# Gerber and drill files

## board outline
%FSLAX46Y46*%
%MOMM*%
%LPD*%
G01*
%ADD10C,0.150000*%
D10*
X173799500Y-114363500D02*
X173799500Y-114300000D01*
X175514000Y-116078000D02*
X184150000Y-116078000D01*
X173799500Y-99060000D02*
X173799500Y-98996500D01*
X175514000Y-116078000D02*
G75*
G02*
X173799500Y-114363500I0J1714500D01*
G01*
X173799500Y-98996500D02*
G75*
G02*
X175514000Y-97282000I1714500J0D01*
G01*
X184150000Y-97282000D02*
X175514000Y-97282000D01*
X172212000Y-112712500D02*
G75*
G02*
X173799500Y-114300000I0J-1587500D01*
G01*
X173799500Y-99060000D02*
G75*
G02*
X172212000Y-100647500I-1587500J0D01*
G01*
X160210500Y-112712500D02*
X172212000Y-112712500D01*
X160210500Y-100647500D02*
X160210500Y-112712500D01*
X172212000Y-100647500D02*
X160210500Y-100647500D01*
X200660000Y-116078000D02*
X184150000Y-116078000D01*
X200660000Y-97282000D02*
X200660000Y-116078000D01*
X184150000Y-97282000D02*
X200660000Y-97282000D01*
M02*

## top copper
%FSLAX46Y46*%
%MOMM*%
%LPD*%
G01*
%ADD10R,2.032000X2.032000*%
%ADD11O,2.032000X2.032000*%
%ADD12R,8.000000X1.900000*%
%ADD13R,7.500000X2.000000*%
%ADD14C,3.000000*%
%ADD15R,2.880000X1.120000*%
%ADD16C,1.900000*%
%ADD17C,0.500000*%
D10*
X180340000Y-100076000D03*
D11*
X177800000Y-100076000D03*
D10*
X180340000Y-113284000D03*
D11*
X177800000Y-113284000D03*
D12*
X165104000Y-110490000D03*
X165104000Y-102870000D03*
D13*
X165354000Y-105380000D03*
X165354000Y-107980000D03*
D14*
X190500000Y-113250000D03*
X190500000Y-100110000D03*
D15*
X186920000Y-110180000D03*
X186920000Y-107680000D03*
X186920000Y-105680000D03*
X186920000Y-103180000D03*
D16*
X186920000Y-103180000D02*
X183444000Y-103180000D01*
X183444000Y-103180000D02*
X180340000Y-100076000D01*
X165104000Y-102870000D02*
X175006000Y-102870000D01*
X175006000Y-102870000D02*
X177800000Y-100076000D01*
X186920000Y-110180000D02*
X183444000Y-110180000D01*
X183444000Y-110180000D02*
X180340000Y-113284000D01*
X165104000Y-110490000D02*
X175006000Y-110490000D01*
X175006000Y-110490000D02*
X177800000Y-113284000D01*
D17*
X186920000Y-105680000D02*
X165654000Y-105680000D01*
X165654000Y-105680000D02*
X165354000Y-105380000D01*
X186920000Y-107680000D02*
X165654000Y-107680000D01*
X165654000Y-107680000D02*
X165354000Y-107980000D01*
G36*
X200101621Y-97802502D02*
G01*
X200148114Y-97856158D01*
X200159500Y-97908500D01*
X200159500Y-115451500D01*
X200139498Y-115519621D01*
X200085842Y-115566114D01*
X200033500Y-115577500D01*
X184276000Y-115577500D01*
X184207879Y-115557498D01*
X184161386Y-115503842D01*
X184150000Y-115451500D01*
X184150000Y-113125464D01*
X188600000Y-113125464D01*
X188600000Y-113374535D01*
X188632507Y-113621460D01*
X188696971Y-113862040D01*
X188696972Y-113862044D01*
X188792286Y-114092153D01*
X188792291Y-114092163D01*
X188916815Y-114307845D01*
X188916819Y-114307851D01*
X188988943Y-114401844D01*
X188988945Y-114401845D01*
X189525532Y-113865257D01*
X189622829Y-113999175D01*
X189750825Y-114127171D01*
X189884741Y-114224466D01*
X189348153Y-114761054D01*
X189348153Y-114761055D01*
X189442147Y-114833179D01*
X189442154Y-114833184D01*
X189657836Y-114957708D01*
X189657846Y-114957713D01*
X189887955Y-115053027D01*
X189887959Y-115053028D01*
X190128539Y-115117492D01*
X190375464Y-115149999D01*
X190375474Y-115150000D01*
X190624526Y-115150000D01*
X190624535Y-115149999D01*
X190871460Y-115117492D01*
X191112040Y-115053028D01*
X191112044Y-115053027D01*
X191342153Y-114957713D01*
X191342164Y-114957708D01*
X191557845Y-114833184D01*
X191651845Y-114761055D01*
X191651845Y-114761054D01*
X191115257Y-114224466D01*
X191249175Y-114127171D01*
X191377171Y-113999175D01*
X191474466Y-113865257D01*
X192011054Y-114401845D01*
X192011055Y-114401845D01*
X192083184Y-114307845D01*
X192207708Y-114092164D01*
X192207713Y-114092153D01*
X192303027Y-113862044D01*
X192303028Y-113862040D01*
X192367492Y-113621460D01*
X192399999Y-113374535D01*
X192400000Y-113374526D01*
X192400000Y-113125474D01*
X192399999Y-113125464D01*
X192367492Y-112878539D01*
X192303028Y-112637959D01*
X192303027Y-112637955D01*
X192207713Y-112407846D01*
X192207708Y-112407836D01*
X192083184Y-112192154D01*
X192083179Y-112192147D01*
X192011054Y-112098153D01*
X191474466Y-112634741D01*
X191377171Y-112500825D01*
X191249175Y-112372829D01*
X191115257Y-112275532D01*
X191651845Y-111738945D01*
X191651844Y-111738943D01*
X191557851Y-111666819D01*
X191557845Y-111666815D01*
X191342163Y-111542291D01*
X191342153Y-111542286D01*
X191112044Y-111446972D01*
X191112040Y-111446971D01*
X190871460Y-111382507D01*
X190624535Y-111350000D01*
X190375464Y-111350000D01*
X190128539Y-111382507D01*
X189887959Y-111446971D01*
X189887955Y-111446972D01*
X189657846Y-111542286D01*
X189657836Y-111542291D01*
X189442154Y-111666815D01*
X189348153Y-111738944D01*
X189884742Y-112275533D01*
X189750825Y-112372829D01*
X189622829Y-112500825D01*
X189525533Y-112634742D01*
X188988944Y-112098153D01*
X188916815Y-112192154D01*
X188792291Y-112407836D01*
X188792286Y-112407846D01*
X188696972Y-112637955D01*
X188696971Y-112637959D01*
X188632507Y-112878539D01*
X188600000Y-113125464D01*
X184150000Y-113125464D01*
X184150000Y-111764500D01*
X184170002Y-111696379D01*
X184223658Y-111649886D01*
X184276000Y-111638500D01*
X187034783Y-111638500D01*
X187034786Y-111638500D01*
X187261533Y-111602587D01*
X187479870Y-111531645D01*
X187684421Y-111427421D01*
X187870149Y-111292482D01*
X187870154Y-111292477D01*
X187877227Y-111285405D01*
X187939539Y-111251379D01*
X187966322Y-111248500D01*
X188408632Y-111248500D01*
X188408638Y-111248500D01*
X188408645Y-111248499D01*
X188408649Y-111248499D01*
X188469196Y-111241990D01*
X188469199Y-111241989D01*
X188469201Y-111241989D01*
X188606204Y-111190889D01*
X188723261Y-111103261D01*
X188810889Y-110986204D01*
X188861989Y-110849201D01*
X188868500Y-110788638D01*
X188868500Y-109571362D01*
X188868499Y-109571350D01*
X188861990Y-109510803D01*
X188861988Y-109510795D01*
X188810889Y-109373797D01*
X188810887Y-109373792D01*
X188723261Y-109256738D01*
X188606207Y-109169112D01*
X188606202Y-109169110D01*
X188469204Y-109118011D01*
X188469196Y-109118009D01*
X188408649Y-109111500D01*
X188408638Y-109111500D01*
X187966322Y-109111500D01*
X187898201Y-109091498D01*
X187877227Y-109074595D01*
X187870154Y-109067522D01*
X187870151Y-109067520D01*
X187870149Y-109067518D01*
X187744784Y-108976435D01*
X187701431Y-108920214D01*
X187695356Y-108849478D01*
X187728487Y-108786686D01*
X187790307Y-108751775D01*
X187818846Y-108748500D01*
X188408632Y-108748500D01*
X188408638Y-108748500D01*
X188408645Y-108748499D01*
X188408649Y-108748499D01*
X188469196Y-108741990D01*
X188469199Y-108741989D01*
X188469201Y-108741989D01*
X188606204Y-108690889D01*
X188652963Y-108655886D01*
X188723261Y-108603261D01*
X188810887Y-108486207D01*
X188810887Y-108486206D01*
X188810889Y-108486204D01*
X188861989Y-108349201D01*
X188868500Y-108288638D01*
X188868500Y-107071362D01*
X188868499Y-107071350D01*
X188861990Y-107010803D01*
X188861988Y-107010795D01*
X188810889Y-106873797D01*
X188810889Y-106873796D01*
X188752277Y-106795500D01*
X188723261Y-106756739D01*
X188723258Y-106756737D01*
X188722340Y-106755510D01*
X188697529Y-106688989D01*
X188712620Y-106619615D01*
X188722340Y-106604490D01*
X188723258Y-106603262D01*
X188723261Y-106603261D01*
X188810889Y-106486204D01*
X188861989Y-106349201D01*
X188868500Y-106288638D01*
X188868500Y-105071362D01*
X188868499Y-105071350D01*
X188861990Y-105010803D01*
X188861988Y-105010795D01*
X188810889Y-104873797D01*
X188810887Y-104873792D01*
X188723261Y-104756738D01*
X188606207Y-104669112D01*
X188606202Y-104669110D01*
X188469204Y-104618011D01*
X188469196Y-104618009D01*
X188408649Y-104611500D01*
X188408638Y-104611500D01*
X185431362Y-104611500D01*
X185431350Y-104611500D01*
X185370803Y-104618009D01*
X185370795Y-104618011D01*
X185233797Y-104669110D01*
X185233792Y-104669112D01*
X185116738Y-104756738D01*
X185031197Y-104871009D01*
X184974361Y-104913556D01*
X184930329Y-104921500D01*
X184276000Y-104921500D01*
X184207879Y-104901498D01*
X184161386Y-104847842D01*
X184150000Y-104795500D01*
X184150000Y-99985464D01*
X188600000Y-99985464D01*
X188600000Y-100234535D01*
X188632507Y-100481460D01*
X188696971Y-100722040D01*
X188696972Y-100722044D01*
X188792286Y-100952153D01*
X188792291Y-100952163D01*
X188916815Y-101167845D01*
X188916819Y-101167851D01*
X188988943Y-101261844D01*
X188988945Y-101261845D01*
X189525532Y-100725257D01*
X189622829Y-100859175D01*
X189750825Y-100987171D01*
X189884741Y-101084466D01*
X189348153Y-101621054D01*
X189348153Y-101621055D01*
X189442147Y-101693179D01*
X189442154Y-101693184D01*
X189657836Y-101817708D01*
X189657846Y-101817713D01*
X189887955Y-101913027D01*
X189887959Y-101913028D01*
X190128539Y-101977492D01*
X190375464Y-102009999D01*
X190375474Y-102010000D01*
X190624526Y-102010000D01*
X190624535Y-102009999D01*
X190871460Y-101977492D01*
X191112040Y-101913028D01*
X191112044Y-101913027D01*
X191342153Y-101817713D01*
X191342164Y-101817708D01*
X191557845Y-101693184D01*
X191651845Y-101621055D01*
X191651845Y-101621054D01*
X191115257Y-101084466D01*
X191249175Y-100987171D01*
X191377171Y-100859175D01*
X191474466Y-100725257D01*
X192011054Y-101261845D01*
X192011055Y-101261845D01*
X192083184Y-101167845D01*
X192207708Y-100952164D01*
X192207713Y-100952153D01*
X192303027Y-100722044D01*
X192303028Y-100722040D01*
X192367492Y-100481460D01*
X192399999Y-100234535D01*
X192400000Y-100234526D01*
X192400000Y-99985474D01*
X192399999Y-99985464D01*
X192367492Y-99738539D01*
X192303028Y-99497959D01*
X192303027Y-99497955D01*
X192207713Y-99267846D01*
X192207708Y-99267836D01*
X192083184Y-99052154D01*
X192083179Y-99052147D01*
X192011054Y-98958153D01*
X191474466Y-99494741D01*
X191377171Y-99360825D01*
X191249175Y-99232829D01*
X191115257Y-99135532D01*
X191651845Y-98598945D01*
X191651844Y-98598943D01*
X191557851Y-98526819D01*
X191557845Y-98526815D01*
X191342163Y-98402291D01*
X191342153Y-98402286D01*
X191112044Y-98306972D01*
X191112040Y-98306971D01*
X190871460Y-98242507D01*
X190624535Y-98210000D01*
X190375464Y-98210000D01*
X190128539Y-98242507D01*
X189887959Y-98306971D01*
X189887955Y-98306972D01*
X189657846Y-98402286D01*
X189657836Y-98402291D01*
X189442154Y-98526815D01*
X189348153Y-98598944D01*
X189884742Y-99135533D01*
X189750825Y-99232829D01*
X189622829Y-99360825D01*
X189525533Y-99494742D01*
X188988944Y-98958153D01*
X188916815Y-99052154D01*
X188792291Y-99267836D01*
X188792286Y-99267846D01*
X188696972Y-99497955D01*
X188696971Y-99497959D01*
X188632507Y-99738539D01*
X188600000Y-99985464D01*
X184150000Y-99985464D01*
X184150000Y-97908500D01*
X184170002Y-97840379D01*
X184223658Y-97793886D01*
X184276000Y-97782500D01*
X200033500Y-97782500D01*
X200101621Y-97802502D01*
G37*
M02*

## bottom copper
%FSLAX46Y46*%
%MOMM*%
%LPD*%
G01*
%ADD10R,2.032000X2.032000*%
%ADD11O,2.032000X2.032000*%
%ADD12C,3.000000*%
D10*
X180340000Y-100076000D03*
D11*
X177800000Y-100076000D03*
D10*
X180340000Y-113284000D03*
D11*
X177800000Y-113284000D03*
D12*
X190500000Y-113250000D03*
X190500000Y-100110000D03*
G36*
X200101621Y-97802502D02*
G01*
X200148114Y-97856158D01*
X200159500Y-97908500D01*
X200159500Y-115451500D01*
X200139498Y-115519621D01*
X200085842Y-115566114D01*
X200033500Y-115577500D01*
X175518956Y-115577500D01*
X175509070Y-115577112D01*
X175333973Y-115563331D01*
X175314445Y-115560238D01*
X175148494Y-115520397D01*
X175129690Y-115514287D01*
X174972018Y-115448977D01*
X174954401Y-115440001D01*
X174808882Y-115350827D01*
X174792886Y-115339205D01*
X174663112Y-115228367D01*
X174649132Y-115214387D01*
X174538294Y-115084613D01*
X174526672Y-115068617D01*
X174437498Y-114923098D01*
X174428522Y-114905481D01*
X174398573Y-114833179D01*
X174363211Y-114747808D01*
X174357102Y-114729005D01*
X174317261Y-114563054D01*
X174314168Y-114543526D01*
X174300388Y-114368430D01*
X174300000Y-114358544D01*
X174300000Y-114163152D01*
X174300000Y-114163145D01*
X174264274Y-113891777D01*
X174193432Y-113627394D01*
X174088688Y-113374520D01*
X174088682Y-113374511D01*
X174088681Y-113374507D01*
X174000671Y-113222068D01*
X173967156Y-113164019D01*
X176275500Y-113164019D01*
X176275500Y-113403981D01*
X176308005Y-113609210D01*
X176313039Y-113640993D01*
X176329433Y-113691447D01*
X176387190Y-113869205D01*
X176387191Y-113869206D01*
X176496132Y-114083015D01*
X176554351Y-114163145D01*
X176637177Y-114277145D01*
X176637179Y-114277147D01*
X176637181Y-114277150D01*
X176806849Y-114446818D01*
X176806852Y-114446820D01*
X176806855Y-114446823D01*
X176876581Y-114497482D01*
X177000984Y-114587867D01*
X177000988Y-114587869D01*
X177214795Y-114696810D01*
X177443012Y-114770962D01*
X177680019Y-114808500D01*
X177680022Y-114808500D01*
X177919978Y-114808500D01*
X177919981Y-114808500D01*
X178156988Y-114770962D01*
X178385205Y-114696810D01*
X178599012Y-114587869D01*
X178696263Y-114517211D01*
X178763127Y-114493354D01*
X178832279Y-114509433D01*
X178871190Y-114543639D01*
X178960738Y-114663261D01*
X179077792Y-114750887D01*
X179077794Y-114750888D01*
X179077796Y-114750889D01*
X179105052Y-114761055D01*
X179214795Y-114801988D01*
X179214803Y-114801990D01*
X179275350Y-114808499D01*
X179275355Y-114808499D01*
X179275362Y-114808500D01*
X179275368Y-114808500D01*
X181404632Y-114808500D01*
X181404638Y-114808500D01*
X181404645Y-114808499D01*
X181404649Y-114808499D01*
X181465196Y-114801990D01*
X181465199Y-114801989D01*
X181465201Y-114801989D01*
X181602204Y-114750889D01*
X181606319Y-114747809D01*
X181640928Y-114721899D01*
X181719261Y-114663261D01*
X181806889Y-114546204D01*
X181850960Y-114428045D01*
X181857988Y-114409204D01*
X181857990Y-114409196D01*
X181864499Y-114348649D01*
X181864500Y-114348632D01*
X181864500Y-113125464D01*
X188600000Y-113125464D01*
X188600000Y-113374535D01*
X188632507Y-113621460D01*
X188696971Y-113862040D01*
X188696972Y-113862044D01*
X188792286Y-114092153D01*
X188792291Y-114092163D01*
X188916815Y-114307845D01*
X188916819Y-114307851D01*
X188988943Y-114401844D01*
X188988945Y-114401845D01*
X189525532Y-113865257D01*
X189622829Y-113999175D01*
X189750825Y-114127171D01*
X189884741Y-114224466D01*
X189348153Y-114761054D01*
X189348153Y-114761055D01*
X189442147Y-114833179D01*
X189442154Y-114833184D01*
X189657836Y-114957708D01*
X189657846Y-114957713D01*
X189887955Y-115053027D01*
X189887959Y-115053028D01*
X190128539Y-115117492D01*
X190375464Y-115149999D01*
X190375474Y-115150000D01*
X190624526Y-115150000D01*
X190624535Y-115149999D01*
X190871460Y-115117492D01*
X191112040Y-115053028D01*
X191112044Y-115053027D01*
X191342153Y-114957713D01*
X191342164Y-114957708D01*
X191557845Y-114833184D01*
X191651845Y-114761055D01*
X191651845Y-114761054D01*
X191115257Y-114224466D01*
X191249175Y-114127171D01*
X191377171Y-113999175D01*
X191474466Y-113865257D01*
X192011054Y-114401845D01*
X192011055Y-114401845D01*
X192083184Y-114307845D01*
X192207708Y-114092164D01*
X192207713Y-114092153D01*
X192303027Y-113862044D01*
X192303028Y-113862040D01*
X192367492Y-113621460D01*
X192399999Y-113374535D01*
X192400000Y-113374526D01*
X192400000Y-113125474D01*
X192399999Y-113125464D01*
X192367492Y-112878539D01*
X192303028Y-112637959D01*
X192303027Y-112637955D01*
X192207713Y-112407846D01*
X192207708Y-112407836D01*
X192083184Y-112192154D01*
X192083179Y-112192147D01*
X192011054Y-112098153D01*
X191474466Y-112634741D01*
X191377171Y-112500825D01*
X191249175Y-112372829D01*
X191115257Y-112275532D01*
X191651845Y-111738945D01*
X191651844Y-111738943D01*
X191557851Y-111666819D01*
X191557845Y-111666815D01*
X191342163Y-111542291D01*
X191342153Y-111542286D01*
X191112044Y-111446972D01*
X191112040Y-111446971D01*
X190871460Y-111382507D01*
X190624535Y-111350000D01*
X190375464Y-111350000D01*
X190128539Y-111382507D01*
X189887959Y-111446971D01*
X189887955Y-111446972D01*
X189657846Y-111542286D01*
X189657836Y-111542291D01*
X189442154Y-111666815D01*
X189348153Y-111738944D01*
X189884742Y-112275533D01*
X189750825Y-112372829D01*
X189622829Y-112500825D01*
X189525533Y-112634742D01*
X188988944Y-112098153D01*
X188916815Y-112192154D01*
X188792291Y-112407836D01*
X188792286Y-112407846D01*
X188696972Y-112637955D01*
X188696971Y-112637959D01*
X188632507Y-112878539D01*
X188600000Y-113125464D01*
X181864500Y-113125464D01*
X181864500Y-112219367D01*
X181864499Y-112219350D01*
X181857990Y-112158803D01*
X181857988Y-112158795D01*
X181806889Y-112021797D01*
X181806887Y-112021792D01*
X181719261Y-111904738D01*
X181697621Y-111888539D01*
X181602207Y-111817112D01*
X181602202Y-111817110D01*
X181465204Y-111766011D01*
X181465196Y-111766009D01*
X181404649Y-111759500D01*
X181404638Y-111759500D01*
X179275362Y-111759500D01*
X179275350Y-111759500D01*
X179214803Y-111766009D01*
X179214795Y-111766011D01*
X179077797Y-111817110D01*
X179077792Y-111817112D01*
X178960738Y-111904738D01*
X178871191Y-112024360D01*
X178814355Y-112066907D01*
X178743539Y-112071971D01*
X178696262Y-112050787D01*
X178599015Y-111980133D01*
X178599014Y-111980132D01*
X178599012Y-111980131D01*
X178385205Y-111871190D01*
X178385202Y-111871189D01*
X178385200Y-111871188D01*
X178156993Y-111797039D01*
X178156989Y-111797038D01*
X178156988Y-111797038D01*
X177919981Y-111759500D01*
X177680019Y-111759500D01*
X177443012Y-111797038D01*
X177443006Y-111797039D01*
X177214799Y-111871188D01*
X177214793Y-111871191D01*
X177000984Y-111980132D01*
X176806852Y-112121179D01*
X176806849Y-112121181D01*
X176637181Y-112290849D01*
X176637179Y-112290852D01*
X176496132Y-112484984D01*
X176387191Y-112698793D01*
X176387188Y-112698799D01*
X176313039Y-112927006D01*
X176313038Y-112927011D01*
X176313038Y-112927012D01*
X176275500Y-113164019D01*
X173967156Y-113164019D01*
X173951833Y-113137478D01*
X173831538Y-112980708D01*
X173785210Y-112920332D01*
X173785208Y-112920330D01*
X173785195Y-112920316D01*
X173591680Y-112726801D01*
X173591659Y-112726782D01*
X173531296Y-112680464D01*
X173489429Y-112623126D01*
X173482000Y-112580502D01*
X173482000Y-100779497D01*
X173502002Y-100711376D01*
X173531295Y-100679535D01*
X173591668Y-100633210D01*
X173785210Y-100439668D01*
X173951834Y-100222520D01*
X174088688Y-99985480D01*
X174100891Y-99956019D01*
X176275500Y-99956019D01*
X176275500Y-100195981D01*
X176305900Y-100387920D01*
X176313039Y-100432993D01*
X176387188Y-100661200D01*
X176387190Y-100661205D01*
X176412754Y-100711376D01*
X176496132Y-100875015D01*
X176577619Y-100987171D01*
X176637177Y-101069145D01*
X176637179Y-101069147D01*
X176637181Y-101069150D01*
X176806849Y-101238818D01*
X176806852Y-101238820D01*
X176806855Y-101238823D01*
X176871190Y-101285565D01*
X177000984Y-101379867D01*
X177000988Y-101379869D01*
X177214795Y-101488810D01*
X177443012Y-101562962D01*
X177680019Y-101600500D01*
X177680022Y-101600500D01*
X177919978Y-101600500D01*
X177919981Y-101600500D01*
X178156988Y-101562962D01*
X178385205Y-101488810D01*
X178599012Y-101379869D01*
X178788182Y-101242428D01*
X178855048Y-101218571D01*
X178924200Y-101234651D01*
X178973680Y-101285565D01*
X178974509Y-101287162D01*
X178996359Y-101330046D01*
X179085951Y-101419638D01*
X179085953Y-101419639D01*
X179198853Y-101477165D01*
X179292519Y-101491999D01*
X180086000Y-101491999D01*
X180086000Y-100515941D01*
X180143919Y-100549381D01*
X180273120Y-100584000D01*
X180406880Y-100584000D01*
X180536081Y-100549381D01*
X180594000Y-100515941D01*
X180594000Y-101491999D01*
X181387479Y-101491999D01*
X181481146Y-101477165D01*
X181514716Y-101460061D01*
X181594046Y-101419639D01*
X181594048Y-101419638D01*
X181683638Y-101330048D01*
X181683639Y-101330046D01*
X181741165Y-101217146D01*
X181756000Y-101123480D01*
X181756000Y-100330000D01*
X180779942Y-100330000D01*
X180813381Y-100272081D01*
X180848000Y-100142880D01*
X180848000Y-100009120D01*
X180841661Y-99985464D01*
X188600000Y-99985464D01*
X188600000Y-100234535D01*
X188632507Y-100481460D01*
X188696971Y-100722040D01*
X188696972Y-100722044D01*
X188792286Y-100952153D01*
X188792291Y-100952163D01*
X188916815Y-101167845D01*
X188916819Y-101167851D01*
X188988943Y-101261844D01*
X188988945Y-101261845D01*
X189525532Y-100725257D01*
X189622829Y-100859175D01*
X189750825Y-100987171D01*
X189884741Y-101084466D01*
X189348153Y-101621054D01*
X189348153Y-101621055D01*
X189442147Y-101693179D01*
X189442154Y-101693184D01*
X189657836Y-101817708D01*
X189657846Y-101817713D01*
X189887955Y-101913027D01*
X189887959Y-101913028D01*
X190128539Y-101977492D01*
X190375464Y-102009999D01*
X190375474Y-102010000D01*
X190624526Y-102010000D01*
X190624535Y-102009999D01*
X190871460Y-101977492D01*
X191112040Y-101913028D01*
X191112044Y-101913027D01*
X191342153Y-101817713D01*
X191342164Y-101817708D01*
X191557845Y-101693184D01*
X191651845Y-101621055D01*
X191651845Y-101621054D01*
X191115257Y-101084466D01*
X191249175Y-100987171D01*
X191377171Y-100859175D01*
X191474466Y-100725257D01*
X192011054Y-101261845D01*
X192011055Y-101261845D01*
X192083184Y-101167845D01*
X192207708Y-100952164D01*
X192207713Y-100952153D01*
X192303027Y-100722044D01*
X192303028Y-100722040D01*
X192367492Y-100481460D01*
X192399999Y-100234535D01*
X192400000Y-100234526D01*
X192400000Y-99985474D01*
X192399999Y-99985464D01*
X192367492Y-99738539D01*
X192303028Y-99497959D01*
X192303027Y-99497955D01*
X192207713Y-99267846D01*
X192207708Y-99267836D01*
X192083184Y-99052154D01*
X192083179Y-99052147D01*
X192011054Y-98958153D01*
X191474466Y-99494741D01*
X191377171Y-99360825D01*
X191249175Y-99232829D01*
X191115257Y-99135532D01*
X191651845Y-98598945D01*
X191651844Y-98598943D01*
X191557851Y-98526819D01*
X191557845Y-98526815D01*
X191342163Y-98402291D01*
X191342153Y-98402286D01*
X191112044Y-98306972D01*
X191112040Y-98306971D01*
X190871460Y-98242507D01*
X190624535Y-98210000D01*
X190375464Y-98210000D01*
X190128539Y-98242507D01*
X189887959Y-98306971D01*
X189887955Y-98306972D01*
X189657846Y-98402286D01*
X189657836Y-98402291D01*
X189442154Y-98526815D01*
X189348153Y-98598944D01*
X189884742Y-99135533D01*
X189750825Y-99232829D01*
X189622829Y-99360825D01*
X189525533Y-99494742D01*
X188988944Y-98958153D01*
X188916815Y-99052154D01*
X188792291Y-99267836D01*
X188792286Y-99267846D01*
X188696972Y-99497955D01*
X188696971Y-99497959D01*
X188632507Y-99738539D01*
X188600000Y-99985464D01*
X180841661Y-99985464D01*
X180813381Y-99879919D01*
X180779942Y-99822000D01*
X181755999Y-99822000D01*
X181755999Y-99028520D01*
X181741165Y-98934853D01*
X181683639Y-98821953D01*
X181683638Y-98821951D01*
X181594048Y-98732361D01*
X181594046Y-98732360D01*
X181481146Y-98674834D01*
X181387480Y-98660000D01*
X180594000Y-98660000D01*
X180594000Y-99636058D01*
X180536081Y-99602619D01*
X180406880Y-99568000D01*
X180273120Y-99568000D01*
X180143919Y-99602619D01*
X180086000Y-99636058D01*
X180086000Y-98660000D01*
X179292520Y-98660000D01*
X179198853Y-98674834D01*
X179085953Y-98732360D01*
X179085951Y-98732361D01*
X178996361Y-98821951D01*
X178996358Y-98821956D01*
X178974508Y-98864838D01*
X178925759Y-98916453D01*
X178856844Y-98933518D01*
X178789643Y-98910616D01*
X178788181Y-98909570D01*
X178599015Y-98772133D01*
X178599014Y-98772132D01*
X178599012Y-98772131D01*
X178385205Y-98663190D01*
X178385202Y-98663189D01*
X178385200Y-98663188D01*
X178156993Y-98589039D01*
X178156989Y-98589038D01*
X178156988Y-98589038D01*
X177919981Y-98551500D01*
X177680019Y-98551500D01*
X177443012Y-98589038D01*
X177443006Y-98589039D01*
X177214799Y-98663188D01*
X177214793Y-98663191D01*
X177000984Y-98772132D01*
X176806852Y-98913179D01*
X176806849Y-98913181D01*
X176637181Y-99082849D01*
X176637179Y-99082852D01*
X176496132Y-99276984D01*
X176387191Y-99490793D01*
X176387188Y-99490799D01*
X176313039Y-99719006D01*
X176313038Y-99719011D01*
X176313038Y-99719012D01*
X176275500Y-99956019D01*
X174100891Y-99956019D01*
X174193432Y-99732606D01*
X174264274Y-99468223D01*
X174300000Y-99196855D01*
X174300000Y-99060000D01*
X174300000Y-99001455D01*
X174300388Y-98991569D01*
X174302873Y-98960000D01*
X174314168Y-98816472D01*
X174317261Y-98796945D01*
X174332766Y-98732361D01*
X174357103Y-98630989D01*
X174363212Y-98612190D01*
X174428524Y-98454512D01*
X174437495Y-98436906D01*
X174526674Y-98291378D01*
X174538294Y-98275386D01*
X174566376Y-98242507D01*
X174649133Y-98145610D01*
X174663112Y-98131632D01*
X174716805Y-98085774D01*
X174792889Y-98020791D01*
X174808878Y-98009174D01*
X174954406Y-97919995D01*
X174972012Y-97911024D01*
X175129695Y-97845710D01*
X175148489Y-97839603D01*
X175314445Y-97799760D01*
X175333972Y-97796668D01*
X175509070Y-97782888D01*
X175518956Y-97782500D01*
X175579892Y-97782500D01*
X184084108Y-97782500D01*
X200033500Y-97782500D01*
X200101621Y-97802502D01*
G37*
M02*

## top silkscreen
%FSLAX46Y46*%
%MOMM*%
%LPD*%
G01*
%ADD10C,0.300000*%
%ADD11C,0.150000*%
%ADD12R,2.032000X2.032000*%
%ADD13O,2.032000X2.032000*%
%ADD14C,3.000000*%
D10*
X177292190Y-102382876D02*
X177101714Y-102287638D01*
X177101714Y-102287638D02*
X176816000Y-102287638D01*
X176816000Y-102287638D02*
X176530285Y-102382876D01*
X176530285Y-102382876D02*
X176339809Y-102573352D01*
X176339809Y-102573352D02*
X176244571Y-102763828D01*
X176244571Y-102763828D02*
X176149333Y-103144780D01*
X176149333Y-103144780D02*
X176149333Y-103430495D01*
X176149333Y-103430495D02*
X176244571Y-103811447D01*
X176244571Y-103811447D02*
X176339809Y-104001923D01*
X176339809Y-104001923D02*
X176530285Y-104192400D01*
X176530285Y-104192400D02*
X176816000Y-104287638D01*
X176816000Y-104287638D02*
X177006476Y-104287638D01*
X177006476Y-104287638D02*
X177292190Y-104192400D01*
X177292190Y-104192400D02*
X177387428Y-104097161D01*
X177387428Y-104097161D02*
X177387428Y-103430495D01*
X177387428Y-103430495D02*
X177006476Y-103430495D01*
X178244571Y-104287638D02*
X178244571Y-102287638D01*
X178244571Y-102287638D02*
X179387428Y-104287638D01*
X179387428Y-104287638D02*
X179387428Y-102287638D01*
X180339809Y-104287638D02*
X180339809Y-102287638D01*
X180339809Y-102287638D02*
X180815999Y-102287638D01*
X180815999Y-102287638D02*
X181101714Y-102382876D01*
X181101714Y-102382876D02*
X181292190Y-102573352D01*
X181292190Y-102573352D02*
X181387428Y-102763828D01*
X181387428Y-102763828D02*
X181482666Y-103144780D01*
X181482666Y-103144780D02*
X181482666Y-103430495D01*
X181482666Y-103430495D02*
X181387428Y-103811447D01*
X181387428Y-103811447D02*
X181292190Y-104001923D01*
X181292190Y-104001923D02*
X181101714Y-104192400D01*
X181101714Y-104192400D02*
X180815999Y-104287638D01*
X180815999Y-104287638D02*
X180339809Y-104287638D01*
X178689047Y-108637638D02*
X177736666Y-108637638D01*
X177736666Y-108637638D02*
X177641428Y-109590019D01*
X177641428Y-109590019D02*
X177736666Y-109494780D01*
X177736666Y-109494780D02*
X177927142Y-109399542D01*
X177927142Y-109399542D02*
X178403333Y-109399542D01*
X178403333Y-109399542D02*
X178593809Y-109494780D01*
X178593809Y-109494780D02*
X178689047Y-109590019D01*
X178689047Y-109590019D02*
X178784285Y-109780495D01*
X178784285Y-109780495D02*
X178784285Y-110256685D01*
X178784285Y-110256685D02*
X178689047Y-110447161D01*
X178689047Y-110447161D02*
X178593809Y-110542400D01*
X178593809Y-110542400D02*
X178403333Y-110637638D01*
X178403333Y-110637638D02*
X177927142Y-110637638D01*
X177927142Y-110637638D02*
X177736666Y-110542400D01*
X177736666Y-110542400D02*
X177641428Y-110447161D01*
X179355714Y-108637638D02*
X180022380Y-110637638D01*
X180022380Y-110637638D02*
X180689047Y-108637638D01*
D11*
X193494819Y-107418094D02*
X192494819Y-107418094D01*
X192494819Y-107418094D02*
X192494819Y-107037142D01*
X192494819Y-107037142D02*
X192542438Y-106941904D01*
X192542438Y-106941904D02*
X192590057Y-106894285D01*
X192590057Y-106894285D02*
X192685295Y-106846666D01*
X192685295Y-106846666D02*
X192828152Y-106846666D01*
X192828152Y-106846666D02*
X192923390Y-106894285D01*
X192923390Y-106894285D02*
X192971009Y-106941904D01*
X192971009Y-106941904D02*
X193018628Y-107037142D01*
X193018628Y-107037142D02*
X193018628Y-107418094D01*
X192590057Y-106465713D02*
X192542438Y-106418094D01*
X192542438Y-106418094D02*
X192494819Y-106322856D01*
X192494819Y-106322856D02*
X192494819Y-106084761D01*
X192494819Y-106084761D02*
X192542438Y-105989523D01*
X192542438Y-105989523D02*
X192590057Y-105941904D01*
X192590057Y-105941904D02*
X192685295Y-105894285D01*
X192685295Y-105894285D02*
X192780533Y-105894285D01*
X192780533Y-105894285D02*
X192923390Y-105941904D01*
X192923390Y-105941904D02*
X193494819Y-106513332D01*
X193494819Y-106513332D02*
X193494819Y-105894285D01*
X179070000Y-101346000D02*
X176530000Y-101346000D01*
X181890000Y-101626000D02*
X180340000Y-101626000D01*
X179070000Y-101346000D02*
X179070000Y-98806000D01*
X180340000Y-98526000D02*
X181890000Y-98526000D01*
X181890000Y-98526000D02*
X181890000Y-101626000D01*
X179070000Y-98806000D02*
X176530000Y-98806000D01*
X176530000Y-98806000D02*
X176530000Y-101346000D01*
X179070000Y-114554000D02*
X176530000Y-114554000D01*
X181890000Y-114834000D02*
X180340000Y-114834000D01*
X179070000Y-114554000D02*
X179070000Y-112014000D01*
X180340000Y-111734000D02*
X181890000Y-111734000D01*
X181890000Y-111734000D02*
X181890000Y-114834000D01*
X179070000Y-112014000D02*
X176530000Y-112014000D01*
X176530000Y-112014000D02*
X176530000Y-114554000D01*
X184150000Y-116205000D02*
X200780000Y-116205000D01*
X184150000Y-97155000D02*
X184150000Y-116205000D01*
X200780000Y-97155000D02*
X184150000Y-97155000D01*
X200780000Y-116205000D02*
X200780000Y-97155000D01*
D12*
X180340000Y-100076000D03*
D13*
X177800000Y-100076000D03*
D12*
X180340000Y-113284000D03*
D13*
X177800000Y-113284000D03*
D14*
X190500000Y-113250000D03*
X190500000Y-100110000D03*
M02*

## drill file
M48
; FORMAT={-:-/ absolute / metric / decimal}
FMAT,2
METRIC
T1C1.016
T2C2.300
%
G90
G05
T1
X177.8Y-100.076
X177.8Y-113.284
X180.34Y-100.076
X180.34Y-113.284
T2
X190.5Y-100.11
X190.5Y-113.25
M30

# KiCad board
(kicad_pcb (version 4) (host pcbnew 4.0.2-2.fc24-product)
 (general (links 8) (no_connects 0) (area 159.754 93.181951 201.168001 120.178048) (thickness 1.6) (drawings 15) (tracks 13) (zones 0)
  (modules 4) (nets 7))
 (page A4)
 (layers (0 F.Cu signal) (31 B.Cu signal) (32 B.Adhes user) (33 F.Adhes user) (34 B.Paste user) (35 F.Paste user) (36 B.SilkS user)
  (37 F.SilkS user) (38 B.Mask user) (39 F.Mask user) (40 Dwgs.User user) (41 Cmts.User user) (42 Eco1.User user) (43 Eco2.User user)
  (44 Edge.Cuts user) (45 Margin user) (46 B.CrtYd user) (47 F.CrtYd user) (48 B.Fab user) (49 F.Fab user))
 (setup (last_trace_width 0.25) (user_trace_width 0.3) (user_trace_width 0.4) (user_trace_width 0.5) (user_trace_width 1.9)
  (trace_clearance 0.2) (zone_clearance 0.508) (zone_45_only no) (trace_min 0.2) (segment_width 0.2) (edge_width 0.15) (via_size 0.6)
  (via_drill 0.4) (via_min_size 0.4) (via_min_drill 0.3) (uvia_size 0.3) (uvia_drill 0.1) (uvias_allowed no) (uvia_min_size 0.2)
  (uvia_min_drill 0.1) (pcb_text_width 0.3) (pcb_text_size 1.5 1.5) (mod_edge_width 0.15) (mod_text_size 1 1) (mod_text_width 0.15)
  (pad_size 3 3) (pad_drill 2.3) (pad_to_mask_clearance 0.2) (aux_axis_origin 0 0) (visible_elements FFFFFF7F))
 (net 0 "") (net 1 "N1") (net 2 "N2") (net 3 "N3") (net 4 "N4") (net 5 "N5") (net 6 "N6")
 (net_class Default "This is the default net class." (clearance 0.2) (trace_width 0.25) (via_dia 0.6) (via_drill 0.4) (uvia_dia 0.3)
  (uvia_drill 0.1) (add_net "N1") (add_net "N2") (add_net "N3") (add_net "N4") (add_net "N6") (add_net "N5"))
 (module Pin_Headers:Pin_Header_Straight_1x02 (layer F.Cu) (at 180.34 100.076 270)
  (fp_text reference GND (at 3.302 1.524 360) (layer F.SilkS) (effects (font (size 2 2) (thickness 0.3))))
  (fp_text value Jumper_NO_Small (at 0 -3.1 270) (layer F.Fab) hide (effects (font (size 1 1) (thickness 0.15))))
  (fp_line (start 1.27 1.27) (end 1.27 3.81) (layer F.SilkS) (width 0.15))
  (fp_line (start 1.55 -1.55) (end 1.55 0) (layer F.SilkS) (width 0.15))
  (fp_line (start 1.27 1.27) (end -1.27 1.27) (layer F.SilkS) (width 0.15))
  (fp_line (start -1.55 0) (end -1.55 -1.55) (layer F.SilkS) (width 0.15))
  (fp_line (start -1.55 -1.55) (end 1.55 -1.55) (layer F.SilkS) (width 0.15))
  (fp_line (start -1.27 1.27) (end -1.27 3.81) (layer F.SilkS) (width 0.15))
  (fp_line (start -1.27 3.81) (end 1.27 3.81) (layer F.SilkS) (width 0.15))
  (pad 1 thru_hole rect (at 0 0 270) (size 2.032 2.032) (drill 1.016) (layers *.Cu *.Mask F.SilkS) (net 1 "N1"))
  (pad 2 thru_hole oval (at 0 2.54 270) (size 2.032 2.032) (drill 1.016) (layers *.Cu *.Mask F.SilkS) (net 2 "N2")))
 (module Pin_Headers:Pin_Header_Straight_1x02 (layer F.Cu) (at 180.34 113.284 270)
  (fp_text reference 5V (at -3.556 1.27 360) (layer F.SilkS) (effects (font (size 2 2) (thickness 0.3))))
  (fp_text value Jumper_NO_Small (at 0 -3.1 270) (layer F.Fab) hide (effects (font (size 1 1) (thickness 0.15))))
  (fp_line (start 1.27 1.27) (end 1.27 3.81) (layer F.SilkS) (width 0.15))
  (fp_line (start 1.55 -1.55) (end 1.55 0) (layer F.SilkS) (width 0.15))
  (fp_line (start 1.27 1.27) (end -1.27 1.27) (layer F.SilkS) (width 0.15))
  (fp_line (start -1.55 0) (end -1.55 -1.55) (layer F.SilkS) (width 0.15))
  (fp_line (start -1.55 -1.55) (end 1.55 -1.55) (layer F.SilkS) (width 0.15))
  (fp_line (start -1.27 1.27) (end -1.27 3.81) (layer F.SilkS) (width 0.15))
  (fp_line (start -1.27 3.81) (end 1.27 3.81) (layer F.SilkS) (width 0.15))
  (pad 1 thru_hole rect (at 0 0 270) (size 2.032 2.032) (drill 1.016) (layers *.Cu *.Mask F.SilkS) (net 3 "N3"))
  (pad 2 thru_hole oval (at 0 2.54 270) (size 2.032 2.032) (drill 1.016) (layers *.Cu *.Mask F.SilkS) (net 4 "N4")))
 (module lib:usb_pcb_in (layer F.Cu) (at 160.204 106.68 270)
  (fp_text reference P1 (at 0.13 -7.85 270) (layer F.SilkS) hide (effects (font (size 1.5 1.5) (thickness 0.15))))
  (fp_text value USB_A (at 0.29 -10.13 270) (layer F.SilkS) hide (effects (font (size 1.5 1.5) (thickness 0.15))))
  (pad 1 connect rect (at 3.81 -4.9 270) (size 1.9 8) (layers F.Cu F.Mask) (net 4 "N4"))
  (pad 4 connect rect (at -3.81 -4.9 270) (size 1.9 8) (layers F.Cu F.Mask) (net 2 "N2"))
  (pad 3 connect rect (at -1.3 -5.15 270) (size 2 7.5) (layers F.Cu F.Mask) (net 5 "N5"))
  (pad 2 connect rect (at 1.3 -5.15 270) (size 2 7.5) (layers F.Cu F.Mask) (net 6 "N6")))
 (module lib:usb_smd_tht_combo (layer F.Cu) (at 190.5 106.68 90)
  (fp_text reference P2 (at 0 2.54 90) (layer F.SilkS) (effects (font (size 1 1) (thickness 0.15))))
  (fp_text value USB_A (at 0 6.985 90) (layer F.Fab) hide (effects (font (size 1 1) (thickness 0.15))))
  (fp_line (start -9.525 -6.35) (end -9.525 10.28) (layer F.SilkS) (width 0.15))
  (fp_line (start 9.525 -6.35) (end -9.525 -6.35) (layer F.SilkS) (width 0.15))
  (fp_line (start 9.525 10.28) (end 9.525 -6.35) (layer F.SilkS) (width 0.15))
  (fp_line (start -9.525 10.28) (end 9.525 10.28) (layer F.SilkS) (width 0.15))
  (pad 5 thru_hole circle (at -6.57 0 90) (size 3 3) (drill 2.3) (layers *.Cu *.Mask F.SilkS) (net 1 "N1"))
  (pad 6 thru_hole circle (at 6.57 0 90) (size 3 3) (drill 2.3) (layers *.Cu *.Mask F.SilkS) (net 1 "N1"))
  (pad 1 smd rect (at -3.5 -3.58 90) (size 1.12 2.88) (layers F.Cu F.Paste F.Mask) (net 3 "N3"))
  (pad 2 smd rect (at -1 -3.58 90) (size 1.12 2.88) (layers F.Cu F.Paste F.Mask) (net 6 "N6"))
  (pad 3 smd rect (at 1 -3.58 90) (size 1.12 2.88) (layers F.Cu F.Paste F.Mask) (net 5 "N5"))
  (pad 4 smd rect (at 3.5 -3.58 90) (size 1.12 2.88) (layers F.Cu F.Paste F.Mask) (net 1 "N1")))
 (gr_line (start 173.7995 114.3635) (end 173.7995 114.3) (layer Edge.Cuts) (width 0.15))
 (gr_line (start 175.514 116.078) (end 184.15 116.078) (layer Edge.Cuts) (width 0.15))
 (gr_line (start 173.7995 99.06) (end 173.7995 98.9965) (layer Edge.Cuts) (width 0.15))
 (gr_arc (start 175.514 114.3635) (end 175.514 116.078) (angle 90) (layer Edge.Cuts) (width 0.15))
 (gr_arc (start 175.514 98.9965) (end 173.7995 98.9965) (angle 90) (layer Edge.Cuts) (width 0.15))
 (gr_line (start 184.15 97.282) (end 175.514 97.282) (layer Edge.Cuts) (width 0.15))
 (gr_arc (start 172.212 114.3) (end 172.212 112.7125) (angle 90) (layer Edge.Cuts) (width 0.15))
 (gr_arc (start 172.212 99.06) (end 173.7995 99.06) (angle 90) (layer Edge.Cuts) (width 0.15))
 (gr_line (start 160.2105 112.7125) (end 172.212 112.7125) (layer Edge.Cuts) (width 0.15))
 (gr_line (start 160.2105 100.6475) (end 160.2105 112.7125) (layer Edge.Cuts) (width 0.15))
 (gr_line (start 172.212 100.6475) (end 160.2105 100.6475) (layer Edge.Cuts) (width 0.15))
 (gr_line (start 200.66 116.078) (end 184.15 116.078) (layer Edge.Cuts) (width 0.15))
 (gr_line (start 200.66 97.282) (end 200.66 116.078) (layer Edge.Cuts) (width 0.15))
 (gr_line (start 184.15 97.282) (end 200.66 97.282) (layer Edge.Cuts) (width 0.15))
 (segment (start 184.15 97.282) (end 200.66 97.282) (width 0.25) (layer Dwgs.User) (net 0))
 (segment (start 186.92 103.18) (end 183.444 103.18) (width 1.9) (layer F.Cu) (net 1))
 (segment (start 183.444 103.18) (end 180.34 100.076) (width 1.9) (layer F.Cu) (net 1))
 (segment (start 165.104 102.87) (end 175.006 102.87) (width 1.9) (layer F.Cu) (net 2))
 (segment (start 175.006 102.87) (end 177.8 100.076) (width 1.9) (layer F.Cu) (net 2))
 (segment (start 186.92 110.18) (end 183.444 110.18) (width 1.9) (layer F.Cu) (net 3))
 (segment (start 183.444 110.18) (end 180.34 113.284) (width 1.9) (layer F.Cu) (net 3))
 (segment (start 165.104 110.49) (end 175.006 110.49) (width 1.9) (layer F.Cu) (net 4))
 (segment (start 175.006 110.49) (end 177.8 113.284) (width 1.9) (layer F.Cu) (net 4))
 (segment (start 186.92 105.68) (end 165.654 105.68) (width 0.5) (layer F.Cu) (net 5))
 (segment (start 165.654 105.68) (end 165.354 105.38) (width 0.5) (layer F.Cu) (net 5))
 (segment (start 186.92 107.68) (end 165.654 107.68) (width 0.5) (layer F.Cu) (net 6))
 (segment (start 165.654 107.68) (end 165.354 107.98) (width 0.5) (layer F.Cu) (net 6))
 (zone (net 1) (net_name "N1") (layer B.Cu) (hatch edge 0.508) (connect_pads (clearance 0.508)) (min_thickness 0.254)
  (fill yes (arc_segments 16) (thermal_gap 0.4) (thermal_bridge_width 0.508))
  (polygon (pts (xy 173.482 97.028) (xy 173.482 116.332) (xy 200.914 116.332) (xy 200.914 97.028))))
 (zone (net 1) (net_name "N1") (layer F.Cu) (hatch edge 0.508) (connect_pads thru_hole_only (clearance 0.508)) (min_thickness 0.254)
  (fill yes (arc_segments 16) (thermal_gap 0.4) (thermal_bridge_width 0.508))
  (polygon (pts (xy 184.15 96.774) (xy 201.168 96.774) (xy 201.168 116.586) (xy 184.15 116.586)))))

